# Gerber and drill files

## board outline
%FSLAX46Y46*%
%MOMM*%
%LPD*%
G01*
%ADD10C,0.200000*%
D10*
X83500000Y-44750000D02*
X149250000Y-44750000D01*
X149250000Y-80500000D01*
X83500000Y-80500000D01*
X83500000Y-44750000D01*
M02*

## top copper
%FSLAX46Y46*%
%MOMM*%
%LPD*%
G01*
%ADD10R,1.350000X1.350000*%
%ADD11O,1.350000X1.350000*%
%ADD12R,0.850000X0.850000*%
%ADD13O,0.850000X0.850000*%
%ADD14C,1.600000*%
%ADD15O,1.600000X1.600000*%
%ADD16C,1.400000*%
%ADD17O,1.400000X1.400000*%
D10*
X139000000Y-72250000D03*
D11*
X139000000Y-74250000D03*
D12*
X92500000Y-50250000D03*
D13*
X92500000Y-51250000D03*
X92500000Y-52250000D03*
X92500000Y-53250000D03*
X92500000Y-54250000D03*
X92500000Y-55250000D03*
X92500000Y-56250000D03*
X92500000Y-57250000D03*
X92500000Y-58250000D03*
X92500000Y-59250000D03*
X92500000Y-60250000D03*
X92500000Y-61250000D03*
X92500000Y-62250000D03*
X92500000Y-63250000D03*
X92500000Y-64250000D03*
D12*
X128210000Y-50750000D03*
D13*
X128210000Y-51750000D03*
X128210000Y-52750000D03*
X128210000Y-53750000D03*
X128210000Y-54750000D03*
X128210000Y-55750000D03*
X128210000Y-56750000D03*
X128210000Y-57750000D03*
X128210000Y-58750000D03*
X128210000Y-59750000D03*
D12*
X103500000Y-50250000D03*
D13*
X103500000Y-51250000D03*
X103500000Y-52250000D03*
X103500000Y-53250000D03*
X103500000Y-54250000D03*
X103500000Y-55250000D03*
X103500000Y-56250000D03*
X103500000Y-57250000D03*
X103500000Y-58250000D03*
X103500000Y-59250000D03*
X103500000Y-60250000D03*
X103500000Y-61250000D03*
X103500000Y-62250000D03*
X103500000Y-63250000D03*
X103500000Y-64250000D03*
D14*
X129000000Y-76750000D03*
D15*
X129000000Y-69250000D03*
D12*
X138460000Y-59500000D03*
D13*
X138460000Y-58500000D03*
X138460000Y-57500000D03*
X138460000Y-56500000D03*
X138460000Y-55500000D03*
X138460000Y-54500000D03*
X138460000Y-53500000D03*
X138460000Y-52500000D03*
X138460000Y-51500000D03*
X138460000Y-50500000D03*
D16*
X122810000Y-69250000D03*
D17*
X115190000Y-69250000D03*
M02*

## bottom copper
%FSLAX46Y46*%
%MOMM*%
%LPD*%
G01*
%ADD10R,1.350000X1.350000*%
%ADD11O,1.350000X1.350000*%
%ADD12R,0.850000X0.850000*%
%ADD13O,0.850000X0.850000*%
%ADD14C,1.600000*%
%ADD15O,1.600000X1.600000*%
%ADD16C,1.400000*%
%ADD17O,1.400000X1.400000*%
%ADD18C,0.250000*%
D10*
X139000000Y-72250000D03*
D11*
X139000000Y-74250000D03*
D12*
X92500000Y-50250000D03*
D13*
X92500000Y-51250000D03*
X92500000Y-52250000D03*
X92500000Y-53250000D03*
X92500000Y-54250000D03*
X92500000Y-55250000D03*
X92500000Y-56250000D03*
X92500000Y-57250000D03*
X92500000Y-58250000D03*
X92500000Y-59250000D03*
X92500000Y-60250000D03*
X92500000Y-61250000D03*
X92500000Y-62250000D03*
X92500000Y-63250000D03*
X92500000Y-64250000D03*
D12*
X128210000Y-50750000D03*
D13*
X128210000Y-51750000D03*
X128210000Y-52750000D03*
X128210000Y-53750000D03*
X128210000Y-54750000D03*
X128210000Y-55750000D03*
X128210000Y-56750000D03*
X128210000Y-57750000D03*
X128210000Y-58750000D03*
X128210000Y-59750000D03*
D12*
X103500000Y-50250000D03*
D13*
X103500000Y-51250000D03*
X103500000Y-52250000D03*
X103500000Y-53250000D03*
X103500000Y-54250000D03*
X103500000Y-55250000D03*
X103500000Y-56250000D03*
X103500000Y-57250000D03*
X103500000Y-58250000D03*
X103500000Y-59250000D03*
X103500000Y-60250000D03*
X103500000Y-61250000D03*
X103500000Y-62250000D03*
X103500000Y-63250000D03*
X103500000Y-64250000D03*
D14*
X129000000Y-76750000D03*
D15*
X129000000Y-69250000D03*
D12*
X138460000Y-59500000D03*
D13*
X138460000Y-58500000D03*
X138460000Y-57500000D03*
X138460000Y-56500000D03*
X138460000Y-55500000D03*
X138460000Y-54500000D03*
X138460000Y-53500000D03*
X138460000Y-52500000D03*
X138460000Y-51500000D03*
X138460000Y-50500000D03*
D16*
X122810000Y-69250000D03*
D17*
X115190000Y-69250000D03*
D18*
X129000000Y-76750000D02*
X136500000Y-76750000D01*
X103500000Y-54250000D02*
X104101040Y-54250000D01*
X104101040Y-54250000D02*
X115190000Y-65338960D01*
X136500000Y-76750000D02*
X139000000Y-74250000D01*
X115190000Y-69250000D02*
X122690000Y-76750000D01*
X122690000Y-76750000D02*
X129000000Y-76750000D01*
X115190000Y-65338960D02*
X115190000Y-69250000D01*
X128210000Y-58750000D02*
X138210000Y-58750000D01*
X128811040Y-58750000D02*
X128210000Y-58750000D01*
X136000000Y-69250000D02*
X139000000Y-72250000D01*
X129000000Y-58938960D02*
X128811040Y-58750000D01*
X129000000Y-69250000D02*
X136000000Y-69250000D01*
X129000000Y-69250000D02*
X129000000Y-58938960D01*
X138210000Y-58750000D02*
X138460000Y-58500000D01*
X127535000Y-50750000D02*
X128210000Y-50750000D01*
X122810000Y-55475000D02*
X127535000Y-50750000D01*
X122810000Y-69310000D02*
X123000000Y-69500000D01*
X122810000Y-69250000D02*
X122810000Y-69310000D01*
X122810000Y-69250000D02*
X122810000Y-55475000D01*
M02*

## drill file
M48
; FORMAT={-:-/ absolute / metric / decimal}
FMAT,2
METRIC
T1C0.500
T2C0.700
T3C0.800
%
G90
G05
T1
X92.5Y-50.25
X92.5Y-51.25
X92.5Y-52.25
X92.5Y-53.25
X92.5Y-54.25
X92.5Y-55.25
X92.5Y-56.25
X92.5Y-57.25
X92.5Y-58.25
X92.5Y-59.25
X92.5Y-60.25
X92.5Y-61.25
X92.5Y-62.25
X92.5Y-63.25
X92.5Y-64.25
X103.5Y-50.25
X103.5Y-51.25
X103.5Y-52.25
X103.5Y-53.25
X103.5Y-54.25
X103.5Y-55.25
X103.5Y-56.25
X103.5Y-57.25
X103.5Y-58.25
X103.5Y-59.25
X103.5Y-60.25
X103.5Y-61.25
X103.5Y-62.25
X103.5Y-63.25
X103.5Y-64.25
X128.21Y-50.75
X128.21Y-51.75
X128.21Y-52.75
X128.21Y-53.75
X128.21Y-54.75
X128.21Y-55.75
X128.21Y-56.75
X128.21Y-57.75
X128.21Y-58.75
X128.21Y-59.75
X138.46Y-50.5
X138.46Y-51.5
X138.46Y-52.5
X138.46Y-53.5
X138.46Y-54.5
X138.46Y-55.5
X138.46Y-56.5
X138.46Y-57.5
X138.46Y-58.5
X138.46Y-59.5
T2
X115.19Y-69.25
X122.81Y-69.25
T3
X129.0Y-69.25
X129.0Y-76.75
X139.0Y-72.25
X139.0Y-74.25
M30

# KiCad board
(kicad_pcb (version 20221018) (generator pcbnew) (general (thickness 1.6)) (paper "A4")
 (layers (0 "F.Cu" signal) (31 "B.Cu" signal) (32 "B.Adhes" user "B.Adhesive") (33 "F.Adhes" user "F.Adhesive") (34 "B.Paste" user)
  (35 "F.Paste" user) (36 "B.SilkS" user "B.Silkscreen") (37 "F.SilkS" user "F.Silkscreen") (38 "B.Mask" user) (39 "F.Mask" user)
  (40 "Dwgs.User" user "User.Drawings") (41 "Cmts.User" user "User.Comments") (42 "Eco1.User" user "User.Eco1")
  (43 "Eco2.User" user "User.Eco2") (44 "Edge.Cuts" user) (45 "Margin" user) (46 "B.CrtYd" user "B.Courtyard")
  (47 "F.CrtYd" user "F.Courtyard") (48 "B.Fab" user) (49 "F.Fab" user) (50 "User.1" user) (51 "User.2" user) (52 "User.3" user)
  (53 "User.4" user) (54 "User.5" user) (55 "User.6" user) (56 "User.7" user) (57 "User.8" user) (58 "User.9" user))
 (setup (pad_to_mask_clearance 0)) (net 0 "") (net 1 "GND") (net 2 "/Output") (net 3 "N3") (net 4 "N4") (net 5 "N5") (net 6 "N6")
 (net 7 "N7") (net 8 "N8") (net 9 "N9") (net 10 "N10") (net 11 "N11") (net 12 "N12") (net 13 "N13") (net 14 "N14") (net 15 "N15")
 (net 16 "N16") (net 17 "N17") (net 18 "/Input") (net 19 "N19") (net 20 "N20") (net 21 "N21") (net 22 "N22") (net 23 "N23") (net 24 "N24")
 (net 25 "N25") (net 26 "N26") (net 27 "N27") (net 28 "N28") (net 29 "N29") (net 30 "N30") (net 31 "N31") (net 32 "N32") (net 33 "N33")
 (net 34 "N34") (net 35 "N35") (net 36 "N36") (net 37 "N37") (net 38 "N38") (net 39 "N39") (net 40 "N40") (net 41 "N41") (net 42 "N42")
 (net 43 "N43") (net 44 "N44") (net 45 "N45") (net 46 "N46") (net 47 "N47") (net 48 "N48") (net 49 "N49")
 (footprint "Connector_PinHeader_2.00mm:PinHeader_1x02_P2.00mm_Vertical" (layer "F.Cu") (at 139 72.25)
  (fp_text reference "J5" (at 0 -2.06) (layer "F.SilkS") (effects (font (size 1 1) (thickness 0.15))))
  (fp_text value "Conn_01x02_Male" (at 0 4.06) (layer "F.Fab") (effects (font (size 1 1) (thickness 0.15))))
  (pad "1" thru_hole rect (at 0 0) (size 1.35 1.35) (drill 0.8) (layers "*.Cu" "*.Mask") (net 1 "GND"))
  (pad "2" thru_hole oval (at 0 2) (size 1.35 1.35) (drill 0.8) (layers "*.Cu" "*.Mask") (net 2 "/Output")))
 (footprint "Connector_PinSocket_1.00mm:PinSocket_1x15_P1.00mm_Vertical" (layer "F.Cu") (at 92.5 50.25)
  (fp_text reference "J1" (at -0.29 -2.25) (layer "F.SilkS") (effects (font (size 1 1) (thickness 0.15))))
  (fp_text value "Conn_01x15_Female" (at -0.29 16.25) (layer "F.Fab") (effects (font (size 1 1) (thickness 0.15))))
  (pad "1" thru_hole rect (at 0 0) (size 0.85 0.85) (drill 0.5) (layers "*.Cu" "*.Mask") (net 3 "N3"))
  (pad "2" thru_hole oval (at 0 1) (size 0.85 0.85) (drill 0.5) (layers "*.Cu" "*.Mask") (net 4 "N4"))
  (pad "3" thru_hole oval (at 0 2) (size 0.85 0.85) (drill 0.5) (layers "*.Cu" "*.Mask") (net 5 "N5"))
  (pad "4" thru_hole oval (at 0 3) (size 0.85 0.85) (drill 0.5) (layers "*.Cu" "*.Mask") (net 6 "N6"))
  (pad "5" thru_hole oval (at 0 4) (size 0.85 0.85) (drill 0.5) (layers "*.Cu" "*.Mask") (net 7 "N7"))
  (pad "6" thru_hole oval (at 0 5) (size 0.85 0.85) (drill 0.5) (layers "*.Cu" "*.Mask") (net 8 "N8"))
  (pad "7" thru_hole oval (at 0 6) (size 0.85 0.85) (drill 0.5) (layers "*.Cu" "*.Mask") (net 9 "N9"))
  (pad "8" thru_hole oval (at 0 7) (size 0.85 0.85) (drill 0.5) (layers "*.Cu" "*.Mask") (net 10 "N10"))
  (pad "9" thru_hole oval (at 0 8) (size 0.85 0.85) (drill 0.5) (layers "*.Cu" "*.Mask") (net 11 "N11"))
  (pad "10" thru_hole oval (at 0 9) (size 0.85 0.85) (drill 0.5) (layers "*.Cu" "*.Mask") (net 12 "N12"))
  (pad "11" thru_hole oval (at 0 10) (size 0.85 0.85) (drill 0.5) (layers "*.Cu" "*.Mask") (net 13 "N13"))
  (pad "12" thru_hole oval (at 0 11) (size 0.85 0.85) (drill 0.5) (layers "*.Cu" "*.Mask") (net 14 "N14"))
  (pad "13" thru_hole oval (at 0 12) (size 0.85 0.85) (drill 0.5) (layers "*.Cu" "*.Mask") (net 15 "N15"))
  (pad "14" thru_hole oval (at 0 13) (size 0.85 0.85) (drill 0.5) (layers "*.Cu" "*.Mask") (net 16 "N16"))
  (pad "15" thru_hole oval (at 0 14) (size 0.85 0.85) (drill 0.5) (layers "*.Cu" "*.Mask") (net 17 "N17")))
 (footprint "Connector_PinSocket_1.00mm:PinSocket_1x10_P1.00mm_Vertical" (layer "F.Cu") (at 128.21 50.75)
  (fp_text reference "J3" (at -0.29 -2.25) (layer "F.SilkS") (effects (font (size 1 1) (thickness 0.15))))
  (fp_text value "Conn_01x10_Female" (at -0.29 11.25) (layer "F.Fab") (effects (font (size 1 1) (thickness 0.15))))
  (pad "1" thru_hole rect (at 0 0) (size 0.85 0.85) (drill 0.5) (layers "*.Cu" "*.Mask") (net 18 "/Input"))
  (pad "2" thru_hole oval (at 0 1) (size 0.85 0.85) (drill 0.5) (layers "*.Cu" "*.Mask") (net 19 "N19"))
  (pad "3" thru_hole oval (at 0 2) (size 0.85 0.85) (drill 0.5) (layers "*.Cu" "*.Mask") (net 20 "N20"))
  (pad "4" thru_hole oval (at 0 3) (size 0.85 0.85) (drill 0.5) (layers "*.Cu" "*.Mask") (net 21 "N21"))
  (pad "5" thru_hole oval (at 0 4) (size 0.85 0.85) (drill 0.5) (layers "*.Cu" "*.Mask") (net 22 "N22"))
  (pad "6" thru_hole oval (at 0 5) (size 0.85 0.85) (drill 0.5) (layers "*.Cu" "*.Mask") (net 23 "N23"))
  (pad "7" thru_hole oval (at 0 6) (size 0.85 0.85) (drill 0.5) (layers "*.Cu" "*.Mask") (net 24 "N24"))
  (pad "8" thru_hole oval (at 0 7) (size 0.85 0.85) (drill 0.5) (layers "*.Cu" "*.Mask") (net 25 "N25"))
  (pad "9" thru_hole oval (at 0 8) (size 0.85 0.85) (drill 0.5) (layers "*.Cu" "*.Mask") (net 1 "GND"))
  (pad "10" thru_hole oval (at 0 9) (size 0.85 0.85) (drill 0.5) (layers "*.Cu" "*.Mask") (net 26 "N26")))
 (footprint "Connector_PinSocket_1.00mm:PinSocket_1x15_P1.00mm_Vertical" (layer "F.Cu") (at 103.5 50.25)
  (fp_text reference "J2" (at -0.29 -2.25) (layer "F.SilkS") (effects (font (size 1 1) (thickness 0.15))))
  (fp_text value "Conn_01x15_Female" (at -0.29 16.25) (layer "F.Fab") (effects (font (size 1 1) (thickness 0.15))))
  (pad "1" thru_hole rect (at 0 0) (size 0.85 0.85) (drill 0.5) (layers "*.Cu" "*.Mask") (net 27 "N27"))
  (pad "2" thru_hole oval (at 0 1) (size 0.85 0.85) (drill 0.5) (layers "*.Cu" "*.Mask") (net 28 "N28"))
  (pad "3" thru_hole oval (at 0 2) (size 0.85 0.85) (drill 0.5) (layers "*.Cu" "*.Mask") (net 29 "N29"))
  (pad "4" thru_hole oval (at 0 3) (size 0.85 0.85) (drill 0.5) (layers "*.Cu" "*.Mask") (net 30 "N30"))
  (pad "5" thru_hole oval (at 0 4) (size 0.85 0.85) (drill 0.5) (layers "*.Cu" "*.Mask") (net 2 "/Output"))
  (pad "6" thru_hole oval (at 0 5) (size 0.85 0.85) (drill 0.5) (layers "*.Cu" "*.Mask") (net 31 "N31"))
  (pad "7" thru_hole oval (at 0 6) (size 0.85 0.85) (drill 0.5) (layers "*.Cu" "*.Mask") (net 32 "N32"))
  (pad "8" thru_hole oval (at 0 7) (size 0.85 0.85) (drill 0.5) (layers "*.Cu" "*.Mask") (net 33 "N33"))
  (pad "9" thru_hole oval (at 0 8) (size 0.85 0.85) (drill 0.5) (layers "*.Cu" "*.Mask") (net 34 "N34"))
  (pad "10" thru_hole oval (at 0 9) (size 0.85 0.85) (drill 0.5) (layers "*.Cu" "*.Mask") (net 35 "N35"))
  (pad "11" thru_hole oval (at 0 10) (size 0.85 0.85) (drill 0.5) (layers "*.Cu" "*.Mask") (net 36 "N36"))
  (pad "12" thru_hole oval (at 0 11) (size 0.85 0.85) (drill 0.5) (layers "*.Cu" "*.Mask") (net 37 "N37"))
  (pad "13" thru_hole oval (at 0 12) (size 0.85 0.85) (drill 0.5) (layers "*.Cu" "*.Mask") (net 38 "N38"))
  (pad "14" thru_hole oval (at 0 13) (size 0.85 0.85) (drill 0.5) (layers "*.Cu" "*.Mask") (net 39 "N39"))
  (pad "15" thru_hole oval (at 0 14) (size 0.85 0.85) (drill 0.5) (layers "*.Cu" "*.Mask") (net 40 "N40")))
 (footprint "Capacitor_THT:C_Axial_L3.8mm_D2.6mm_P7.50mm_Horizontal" (layer "F.Cu") (at 129 76.75 90)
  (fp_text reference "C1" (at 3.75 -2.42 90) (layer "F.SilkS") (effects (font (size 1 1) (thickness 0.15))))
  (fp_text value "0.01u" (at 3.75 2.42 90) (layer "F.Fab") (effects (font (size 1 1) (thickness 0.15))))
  (pad "1" thru_hole circle (at 0 0 90) (size 1.6 1.6) (drill 0.8) (layers "*.Cu" "*.Mask") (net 2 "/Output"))
  (pad "2" thru_hole oval (at 7.5 0 90) (size 1.6 1.6) (drill 0.8) (layers "*.Cu" "*.Mask") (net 1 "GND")))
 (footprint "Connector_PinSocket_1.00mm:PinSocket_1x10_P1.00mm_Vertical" (layer "F.Cu") (at 138.46 59.5 180)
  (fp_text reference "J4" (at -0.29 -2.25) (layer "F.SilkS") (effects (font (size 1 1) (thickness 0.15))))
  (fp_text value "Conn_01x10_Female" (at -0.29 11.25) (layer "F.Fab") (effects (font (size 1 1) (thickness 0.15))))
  (pad "1" thru_hole rect (at 0 0 180) (size 0.85 0.85) (drill 0.5) (layers "*.Cu" "*.Mask") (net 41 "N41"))
  (pad "2" thru_hole oval (at 0 1 180) (size 0.85 0.85) (drill 0.5) (layers "*.Cu" "*.Mask") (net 1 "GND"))
  (pad "3" thru_hole oval (at 0 2 180) (size 0.85 0.85) (drill 0.5) (layers "*.Cu" "*.Mask") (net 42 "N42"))
  (pad "4" thru_hole oval (at 0 3 180) (size 0.85 0.85) (drill 0.5) (layers "*.Cu" "*.Mask") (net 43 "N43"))
  (pad "5" thru_hole oval (at 0 4 180) (size 0.85 0.85) (drill 0.5) (layers "*.Cu" "*.Mask") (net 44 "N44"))
  (pad "6" thru_hole oval (at 0 5 180) (size 0.85 0.85) (drill 0.5) (layers "*.Cu" "*.Mask") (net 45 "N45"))
  (pad "7" thru_hole oval (at 0 6 180) (size 0.85 0.85) (drill 0.5) (layers "*.Cu" "*.Mask") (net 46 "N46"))
  (pad "8" thru_hole oval (at 0 7 180) (size 0.85 0.85) (drill 0.5) (layers "*.Cu" "*.Mask") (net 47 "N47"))
  (pad "9" thru_hole oval (at 0 8 180) (size 0.85 0.85) (drill 0.5) (layers "*.Cu" "*.Mask") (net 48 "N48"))
  (pad "10" thru_hole oval (at 0 9 180) (size 0.85 0.85) (drill 0.5) (layers "*.Cu" "*.Mask") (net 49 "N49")))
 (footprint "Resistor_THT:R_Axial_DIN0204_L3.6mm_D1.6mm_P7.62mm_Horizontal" (layer "F.Cu") (at 122.81 69.25 180)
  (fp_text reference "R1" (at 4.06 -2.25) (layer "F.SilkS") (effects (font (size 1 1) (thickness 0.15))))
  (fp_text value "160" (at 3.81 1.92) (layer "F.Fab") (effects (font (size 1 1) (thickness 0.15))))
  (pad "1" thru_hole circle (at 0 0 180) (size 1.4 1.4) (drill 0.7) (layers "*.Cu" "*.Mask") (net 18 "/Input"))
  (pad "2" thru_hole oval (at 7.62 0 180) (size 1.4 1.4) (drill 0.7) (layers "*.Cu" "*.Mask") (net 2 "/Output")))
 (gr_rect (start 83.5 44.75) (end 149.25 80.5) (stroke (width 0.2) (type default)) (fill none) (layer "Edge.Cuts"))
 (segment (start 129 76.75) (end 136.5 76.75) (width 0.25) (layer "B.Cu") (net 2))
 (segment (start 103.5 54.25) (end 104.10104 54.25) (width 0.25) (layer "B.Cu") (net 2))
 (segment (start 104.10104 54.25) (end 115.19 65.33896) (width 0.25) (layer "B.Cu") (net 2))
 (segment (start 136.5 76.75) (end 139 74.25) (width 0.25) (layer "B.Cu") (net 2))
 (segment (start 115.19 69.25) (end 122.69 76.75) (width 0.25) (layer "B.Cu") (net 2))
 (segment (start 122.69 76.75) (end 129 76.75) (width 0.25) (layer "B.Cu") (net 2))
 (segment (start 115.19 65.33896) (end 115.19 69.25) (width 0.25) (layer "B.Cu") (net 2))
 (segment (start 128.21 58.75) (end 138.21 58.75) (width 0.25) (layer "B.Cu") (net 1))
 (segment (start 128.81104 58.75) (end 128.21 58.75) (width 0.25) (layer "B.Cu") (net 1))
 (segment (start 136 69.25) (end 139 72.25) (width 0.25) (layer "B.Cu") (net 1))
 (segment (start 129 58.93896) (end 128.81104 58.75) (width 0.25) (layer "B.Cu") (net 1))
 (segment (start 129 69.25) (end 136 69.25) (width 0.25) (layer "B.Cu") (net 1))
 (segment (start 129 69.25) (end 129 58.93896) (width 0.25) (layer "B.Cu") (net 1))
 (segment (start 138.21 58.75) (end 138.46 58.5) (width 0.25) (layer "B.Cu") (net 1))
 (segment (start 127.535 50.75) (end 128.21 50.75) (width 0.25) (layer "B.Cu") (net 18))
 (segment (start 122.81 55.475) (end 127.535 50.75) (width 0.25) (layer "B.Cu") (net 18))
 (segment (start 122.81 69.31) (end 123 69.5) (width 0.25) (layer "B.Cu") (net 18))
 (segment (start 122.81 69.25) (end 122.81 69.31) (width 0.25) (layer "B.Cu") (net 18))
 (segment (start 122.81 69.25) (end 122.81 55.475) (width 0.25) (layer "B.Cu") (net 18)))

